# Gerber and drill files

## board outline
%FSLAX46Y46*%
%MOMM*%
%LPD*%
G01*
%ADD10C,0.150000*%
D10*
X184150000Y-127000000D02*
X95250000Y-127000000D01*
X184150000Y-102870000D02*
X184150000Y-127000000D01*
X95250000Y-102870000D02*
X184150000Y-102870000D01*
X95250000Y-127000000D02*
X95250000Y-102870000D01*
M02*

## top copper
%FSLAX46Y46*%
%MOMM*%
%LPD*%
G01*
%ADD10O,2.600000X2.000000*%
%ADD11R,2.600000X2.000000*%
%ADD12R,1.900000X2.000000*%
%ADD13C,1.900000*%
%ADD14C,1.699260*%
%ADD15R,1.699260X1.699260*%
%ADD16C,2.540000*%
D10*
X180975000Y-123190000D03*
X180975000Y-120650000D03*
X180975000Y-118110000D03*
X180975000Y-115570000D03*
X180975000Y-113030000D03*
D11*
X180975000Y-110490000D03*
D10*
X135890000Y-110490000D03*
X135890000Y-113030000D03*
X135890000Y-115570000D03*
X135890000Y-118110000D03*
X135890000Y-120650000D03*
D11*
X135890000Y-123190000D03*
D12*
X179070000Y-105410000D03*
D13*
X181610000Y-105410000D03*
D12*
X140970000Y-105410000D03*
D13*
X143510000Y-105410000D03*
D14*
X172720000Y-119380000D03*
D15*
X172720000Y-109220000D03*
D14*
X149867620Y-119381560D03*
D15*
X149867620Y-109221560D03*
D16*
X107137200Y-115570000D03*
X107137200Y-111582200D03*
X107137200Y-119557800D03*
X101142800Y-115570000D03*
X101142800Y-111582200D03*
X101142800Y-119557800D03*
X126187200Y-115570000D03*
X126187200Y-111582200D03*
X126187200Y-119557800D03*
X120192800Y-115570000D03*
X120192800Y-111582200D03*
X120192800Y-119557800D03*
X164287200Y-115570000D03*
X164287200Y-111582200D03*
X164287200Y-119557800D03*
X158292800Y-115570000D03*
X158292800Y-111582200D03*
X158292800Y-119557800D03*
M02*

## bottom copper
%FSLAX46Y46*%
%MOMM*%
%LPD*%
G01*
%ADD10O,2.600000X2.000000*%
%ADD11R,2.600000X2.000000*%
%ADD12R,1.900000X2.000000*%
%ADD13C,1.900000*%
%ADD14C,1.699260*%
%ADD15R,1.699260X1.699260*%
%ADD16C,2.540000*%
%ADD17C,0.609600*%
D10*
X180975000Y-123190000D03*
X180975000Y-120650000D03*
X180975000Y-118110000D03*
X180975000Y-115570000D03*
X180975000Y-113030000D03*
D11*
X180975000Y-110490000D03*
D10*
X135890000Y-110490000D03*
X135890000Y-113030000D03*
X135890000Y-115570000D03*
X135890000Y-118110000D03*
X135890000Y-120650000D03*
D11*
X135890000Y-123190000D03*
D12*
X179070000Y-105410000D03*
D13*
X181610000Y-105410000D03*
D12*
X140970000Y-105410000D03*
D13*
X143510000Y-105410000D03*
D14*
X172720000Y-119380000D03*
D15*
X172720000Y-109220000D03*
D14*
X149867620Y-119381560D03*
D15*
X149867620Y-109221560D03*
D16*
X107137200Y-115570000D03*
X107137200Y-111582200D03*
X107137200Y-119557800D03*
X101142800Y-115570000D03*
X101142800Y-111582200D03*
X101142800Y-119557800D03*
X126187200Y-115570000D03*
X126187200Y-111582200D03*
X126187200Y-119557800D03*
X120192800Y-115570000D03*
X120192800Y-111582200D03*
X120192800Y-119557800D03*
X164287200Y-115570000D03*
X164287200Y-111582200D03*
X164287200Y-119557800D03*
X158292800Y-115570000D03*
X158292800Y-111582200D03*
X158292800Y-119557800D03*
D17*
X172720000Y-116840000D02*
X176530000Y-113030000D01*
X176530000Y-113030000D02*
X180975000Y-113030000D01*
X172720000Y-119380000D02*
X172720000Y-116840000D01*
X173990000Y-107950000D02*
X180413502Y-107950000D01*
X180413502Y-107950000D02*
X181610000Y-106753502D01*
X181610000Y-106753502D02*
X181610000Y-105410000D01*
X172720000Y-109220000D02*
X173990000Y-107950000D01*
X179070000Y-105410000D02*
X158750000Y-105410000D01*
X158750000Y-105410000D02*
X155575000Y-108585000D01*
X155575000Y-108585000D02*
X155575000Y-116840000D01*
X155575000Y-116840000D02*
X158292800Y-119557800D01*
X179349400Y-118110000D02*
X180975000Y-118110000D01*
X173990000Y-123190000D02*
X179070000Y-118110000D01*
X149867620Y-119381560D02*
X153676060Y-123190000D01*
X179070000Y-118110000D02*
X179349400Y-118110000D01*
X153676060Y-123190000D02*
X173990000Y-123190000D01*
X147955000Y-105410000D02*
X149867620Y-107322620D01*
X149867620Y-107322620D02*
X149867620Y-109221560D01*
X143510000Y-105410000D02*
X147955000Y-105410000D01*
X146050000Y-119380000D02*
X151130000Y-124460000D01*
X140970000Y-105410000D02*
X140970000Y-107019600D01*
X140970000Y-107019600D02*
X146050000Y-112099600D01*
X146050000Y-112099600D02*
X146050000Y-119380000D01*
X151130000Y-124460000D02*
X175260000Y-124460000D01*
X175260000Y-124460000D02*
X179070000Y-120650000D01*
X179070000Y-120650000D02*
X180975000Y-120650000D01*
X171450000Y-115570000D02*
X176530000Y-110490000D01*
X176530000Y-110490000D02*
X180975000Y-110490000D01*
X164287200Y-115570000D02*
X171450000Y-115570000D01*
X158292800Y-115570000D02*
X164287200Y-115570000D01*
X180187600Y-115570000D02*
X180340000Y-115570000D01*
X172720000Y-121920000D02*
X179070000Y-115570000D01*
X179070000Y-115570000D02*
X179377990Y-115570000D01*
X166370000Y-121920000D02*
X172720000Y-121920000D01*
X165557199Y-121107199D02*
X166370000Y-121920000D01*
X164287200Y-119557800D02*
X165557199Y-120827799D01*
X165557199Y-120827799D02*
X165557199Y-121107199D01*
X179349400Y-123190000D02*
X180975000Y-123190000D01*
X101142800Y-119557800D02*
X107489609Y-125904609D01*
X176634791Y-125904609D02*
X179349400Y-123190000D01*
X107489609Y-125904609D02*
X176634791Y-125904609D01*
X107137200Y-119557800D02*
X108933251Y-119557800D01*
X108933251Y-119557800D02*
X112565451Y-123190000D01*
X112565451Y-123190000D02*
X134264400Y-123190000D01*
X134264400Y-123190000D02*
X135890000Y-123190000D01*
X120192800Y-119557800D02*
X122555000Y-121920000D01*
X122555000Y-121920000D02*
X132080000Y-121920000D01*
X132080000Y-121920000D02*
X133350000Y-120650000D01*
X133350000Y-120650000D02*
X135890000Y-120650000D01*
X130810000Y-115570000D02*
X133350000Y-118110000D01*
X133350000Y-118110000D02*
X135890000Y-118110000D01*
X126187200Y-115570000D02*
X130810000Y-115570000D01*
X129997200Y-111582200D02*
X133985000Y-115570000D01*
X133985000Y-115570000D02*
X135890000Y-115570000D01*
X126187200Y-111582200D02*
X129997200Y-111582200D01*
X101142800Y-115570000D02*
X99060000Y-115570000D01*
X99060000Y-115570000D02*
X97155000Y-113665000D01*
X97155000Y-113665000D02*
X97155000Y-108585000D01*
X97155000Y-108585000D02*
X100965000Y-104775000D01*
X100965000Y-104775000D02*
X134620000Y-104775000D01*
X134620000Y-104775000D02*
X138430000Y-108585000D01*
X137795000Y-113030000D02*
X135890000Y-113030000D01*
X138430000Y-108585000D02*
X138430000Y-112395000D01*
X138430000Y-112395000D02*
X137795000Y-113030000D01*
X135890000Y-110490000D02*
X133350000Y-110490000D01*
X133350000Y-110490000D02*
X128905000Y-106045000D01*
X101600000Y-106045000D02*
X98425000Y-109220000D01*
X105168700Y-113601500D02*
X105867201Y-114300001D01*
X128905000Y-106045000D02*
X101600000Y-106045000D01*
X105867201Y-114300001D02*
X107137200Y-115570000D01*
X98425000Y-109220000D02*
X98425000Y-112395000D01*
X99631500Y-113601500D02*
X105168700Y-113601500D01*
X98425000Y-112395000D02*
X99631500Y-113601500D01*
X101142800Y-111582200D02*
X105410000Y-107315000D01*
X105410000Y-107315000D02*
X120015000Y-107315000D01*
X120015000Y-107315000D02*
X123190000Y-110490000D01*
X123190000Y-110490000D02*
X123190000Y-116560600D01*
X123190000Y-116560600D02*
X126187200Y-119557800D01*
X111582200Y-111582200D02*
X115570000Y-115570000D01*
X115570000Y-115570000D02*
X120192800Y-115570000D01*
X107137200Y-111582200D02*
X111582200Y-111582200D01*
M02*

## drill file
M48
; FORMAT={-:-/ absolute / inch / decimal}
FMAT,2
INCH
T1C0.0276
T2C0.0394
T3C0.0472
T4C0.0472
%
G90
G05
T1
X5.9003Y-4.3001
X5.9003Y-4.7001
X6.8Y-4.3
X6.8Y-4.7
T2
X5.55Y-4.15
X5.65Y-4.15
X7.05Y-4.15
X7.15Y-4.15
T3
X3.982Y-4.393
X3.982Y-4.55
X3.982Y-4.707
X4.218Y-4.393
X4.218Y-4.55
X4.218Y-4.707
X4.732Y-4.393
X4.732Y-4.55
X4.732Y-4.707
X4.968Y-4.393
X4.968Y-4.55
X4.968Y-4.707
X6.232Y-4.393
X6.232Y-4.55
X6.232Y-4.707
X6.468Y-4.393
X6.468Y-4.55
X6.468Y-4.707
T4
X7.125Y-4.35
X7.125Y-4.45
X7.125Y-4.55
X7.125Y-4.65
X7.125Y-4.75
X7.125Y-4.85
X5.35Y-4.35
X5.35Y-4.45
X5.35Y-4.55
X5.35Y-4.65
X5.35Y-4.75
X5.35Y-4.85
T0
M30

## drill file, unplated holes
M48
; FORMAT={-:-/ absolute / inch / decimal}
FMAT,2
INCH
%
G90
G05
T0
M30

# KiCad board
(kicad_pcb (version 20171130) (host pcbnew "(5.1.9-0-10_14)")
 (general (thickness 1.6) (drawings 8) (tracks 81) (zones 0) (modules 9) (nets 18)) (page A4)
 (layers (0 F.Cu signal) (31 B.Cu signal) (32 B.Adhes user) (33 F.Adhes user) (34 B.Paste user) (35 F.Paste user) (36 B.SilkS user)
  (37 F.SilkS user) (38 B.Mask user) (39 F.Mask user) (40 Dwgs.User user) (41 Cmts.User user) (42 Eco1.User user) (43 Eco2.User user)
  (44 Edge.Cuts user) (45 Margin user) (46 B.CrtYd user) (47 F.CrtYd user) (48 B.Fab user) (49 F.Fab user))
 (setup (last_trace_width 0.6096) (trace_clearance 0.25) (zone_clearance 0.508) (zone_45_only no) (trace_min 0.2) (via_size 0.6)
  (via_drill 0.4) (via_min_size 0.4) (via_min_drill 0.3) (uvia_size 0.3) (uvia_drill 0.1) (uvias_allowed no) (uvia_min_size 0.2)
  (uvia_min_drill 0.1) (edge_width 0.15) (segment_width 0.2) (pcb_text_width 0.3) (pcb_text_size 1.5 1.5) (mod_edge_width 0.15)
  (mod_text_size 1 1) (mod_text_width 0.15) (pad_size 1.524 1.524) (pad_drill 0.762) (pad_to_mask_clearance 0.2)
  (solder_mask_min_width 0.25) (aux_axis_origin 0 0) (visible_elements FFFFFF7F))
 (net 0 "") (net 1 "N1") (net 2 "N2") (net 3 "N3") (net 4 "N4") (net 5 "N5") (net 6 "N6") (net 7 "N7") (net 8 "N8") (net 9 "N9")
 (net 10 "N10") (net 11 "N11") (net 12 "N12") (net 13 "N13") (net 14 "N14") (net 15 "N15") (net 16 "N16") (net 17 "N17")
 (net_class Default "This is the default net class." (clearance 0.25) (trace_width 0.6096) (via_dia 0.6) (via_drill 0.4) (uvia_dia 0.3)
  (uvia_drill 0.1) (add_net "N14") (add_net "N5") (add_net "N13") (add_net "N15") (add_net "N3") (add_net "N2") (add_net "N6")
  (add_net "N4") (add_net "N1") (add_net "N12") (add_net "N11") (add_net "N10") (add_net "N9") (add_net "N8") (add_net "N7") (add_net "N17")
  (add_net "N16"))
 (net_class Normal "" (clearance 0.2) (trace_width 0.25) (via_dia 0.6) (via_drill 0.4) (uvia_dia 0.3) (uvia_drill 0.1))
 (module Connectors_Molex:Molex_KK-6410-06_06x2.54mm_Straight (layer F.Cu) (at 180.975 110.49 270)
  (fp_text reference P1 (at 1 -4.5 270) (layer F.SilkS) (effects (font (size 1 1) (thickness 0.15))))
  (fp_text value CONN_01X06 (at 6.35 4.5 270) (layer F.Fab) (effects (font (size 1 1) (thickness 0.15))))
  (pad 6 thru_hole oval (at 12.7 0 270) (size 2 2.6) (drill 1.2) (layers *.Cu *.Mask) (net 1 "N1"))
  (pad 5 thru_hole oval (at 10.16 0 270) (size 2 2.6) (drill 1.2) (layers *.Cu *.Mask) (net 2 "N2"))
  (pad 4 thru_hole oval (at 7.62 0 270) (size 2 2.6) (drill 1.2) (layers *.Cu *.Mask) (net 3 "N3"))
  (pad 3 thru_hole oval (at 5.08 0 270) (size 2 2.6) (drill 1.2) (layers *.Cu *.Mask) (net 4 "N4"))
  (pad 2 thru_hole oval (at 2.54 0 270) (size 2 2.6) (drill 1.2) (layers *.Cu *.Mask) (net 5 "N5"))
  (pad 1 thru_hole rect (at 0 0 270) (size 2 2.6) (drill 1.2) (layers *.Cu *.Mask) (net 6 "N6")))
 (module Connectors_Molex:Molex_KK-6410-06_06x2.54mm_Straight (layer F.Cu) (at 135.89 123.19 90)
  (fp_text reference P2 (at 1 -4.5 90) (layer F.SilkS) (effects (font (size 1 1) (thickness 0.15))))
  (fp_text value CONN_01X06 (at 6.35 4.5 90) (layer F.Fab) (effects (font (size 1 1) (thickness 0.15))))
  (pad 6 thru_hole oval (at 12.7 0 90) (size 2 2.6) (drill 1.2) (layers *.Cu *.Mask) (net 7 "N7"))
  (pad 5 thru_hole oval (at 10.16 0 90) (size 2 2.6) (drill 1.2) (layers *.Cu *.Mask) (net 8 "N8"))
  (pad 4 thru_hole oval (at 7.62 0 90) (size 2 2.6) (drill 1.2) (layers *.Cu *.Mask) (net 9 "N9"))
  (pad 3 thru_hole oval (at 5.08 0 90) (size 2 2.6) (drill 1.2) (layers *.Cu *.Mask) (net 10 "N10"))
  (pad 2 thru_hole oval (at 2.54 0 90) (size 2 2.6) (drill 1.2) (layers *.Cu *.Mask) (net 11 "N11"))
  (pad 1 thru_hole rect (at 0 0 90) (size 2 2.6) (drill 1.2) (layers *.Cu *.Mask) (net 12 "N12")))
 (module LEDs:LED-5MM (layer F.Cu) (at 179.07 105.41)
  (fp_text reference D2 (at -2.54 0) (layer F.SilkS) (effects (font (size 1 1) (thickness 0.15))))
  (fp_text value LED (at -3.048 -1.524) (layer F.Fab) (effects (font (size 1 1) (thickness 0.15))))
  (pad 1 thru_hole rect (at 0 0 90) (size 2 1.9) (drill 1.00076) (layers *.Cu *.Mask F.SilkS) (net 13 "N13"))
  (pad 2 thru_hole circle (at 2.54 0) (size 1.9 1.9) (drill 1.00076) (layers *.Cu *.Mask F.SilkS) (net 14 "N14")))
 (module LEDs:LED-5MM (layer F.Cu) (at 140.97 105.41)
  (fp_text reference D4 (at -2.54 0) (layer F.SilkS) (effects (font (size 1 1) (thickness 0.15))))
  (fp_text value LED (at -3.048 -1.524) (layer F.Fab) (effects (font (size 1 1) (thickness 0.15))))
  (pad 1 thru_hole rect (at 0 0 90) (size 2 1.9) (drill 1.00076) (layers *.Cu *.Mask F.SilkS) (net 2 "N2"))
  (pad 2 thru_hole circle (at 2.54 0) (size 1.9 1.9) (drill 1.00076) (layers *.Cu *.Mask F.SilkS) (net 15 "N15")))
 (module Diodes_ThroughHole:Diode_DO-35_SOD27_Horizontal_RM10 (layer F.Cu) (at 172.71746 109.21948 270)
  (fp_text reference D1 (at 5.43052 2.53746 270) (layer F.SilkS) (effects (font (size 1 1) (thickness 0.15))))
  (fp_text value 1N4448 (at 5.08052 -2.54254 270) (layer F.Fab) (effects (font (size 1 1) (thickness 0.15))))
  (pad 2 thru_hole circle (at 10.16052 -0.00254 90) (size 1.69926 1.69926) (drill 0.70104) (layers *.Cu *.Mask F.SilkS) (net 5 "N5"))
  (pad 1 thru_hole rect (at 0.00052 -0.00254 90) (size 1.69926 1.69926) (drill 0.70104) (layers *.Cu *.Mask F.SilkS) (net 14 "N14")))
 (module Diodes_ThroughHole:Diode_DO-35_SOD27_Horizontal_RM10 (layer F.Cu) (at 149.86508 109.22104 270)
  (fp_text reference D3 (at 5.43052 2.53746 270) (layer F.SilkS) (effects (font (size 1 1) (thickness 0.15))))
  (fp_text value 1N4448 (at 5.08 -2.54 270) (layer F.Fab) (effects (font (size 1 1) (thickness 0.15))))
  (pad 2 thru_hole circle (at 10.16052 -0.00254 90) (size 1.69926 1.69926) (drill 0.70104) (layers *.Cu *.Mask F.SilkS) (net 3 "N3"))
  (pad 1 thru_hole rect (at 0.00052 -0.00254 90) (size 1.69926 1.69926) (drill 0.70104) (layers *.Cu *.Mask F.SilkS) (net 15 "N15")))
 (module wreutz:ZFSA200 (layer F.Cu) (at 104.14 115.57 270)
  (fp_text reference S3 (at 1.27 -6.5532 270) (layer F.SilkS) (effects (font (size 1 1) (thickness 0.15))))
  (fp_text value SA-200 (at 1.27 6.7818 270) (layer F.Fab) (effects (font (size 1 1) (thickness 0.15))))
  (pad 10 thru_hole circle (at 0 -2.9972 270) (size 2.54 2.54) (drill 1.19888) (layers *.Cu *.Mask F.SilkS) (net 7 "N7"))
  (pad 11 thru_hole circle (at -3.9878 -2.9972 270) (size 2.54 2.54) (drill 1.19888) (layers *.Cu *.Mask F.SilkS) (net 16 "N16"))
  (pad 12 thru_hole circle (at 3.9878 -2.9972 270) (size 2.54 2.54) (drill 1.19888) (layers *.Cu *.Mask F.SilkS) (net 12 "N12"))
  (pad 20 thru_hole circle (at 0 2.9972 270) (size 2.54 2.54) (drill 1.19888) (layers *.Cu *.Mask F.SilkS) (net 8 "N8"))
  (pad 21 thru_hole circle (at -3.9878 2.9972 270) (size 2.54 2.54) (drill 1.19888) (layers *.Cu *.Mask F.SilkS) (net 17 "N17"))
  (pad 22 thru_hole circle (at 3.9878 2.9972 270) (size 2.54 2.54) (drill 1.19888) (layers *.Cu *.Mask F.SilkS) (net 1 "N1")))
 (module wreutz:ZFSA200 (layer F.Cu) (at 123.19 115.57 270)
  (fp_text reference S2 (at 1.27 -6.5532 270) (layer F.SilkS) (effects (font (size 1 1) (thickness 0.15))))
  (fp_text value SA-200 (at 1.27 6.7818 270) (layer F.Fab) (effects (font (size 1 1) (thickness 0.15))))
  (pad 10 thru_hole circle (at 0 -2.9972 270) (size 2.54 2.54) (drill 1.19888) (layers *.Cu *.Mask F.SilkS) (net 10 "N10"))
  (pad 11 thru_hole circle (at -3.9878 -2.9972 270) (size 2.54 2.54) (drill 1.19888) (layers *.Cu *.Mask F.SilkS) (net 9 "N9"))
  (pad 12 thru_hole circle (at 3.9878 -2.9972 270) (size 2.54 2.54) (drill 1.19888) (layers *.Cu *.Mask F.SilkS) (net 17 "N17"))
  (pad 20 thru_hole circle (at 0 2.9972 270) (size 2.54 2.54) (drill 1.19888) (layers *.Cu *.Mask F.SilkS) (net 16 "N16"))
  (pad 21 thru_hole circle (at -3.9878 2.9972 270) (size 2.54 2.54) (drill 1.19888) (layers *.Cu *.Mask F.SilkS))
  (pad 22 thru_hole circle (at 3.9878 2.9972 270) (size 2.54 2.54) (drill 1.19888) (layers *.Cu *.Mask F.SilkS) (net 11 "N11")))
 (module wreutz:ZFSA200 (layer F.Cu) (at 161.29 115.57 270)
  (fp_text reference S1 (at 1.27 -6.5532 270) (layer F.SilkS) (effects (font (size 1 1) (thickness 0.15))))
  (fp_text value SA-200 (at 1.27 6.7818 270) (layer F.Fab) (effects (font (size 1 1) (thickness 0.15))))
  (pad 10 thru_hole circle (at 0 -2.9972 270) (size 2.54 2.54) (drill 1.19888) (layers *.Cu *.Mask F.SilkS) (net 6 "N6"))
  (pad 11 thru_hole circle (at -3.9878 -2.9972 270) (size 2.54 2.54) (drill 1.19888) (layers *.Cu *.Mask F.SilkS))
  (pad 12 thru_hole circle (at 3.9878 -2.9972 270) (size 2.54 2.54) (drill 1.19888) (layers *.Cu *.Mask F.SilkS) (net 4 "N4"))
  (pad 20 thru_hole circle (at 0 2.9972 270) (size 2.54 2.54) (drill 1.19888) (layers *.Cu *.Mask F.SilkS) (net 6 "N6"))
  (pad 21 thru_hole circle (at -3.9878 2.9972 270) (size 2.54 2.54) (drill 1.19888) (layers *.Cu *.Mask F.SilkS))
  (pad 22 thru_hole circle (at 3.9878 2.9972 270) (size 2.54 2.54) (drill 1.19888) (layers *.Cu *.Mask F.SilkS) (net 13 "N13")))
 (gr_line (start 184.15 127) (end 95.25 127) (layer Edge.Cuts) (width 0.15))
 (gr_line (start 184.15 102.87) (end 184.15 127) (layer Edge.Cuts) (width 0.15))
 (gr_line (start 95.25 102.87) (end 184.15 102.87) (layer Edge.Cuts) (width 0.15))
 (gr_line (start 95.25 127) (end 95.25 102.87) (layer Edge.Cuts) (width 0.15))
 (segment (start 172.72 116.84) (end 176.53 113.03) (width 0.6096) (layer B.Cu) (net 5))
 (segment (start 176.53 113.03) (end 180.975 113.03) (width 0.6096) (layer B.Cu) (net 5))
 (segment (start 172.72 119.38) (end 172.72 116.84) (width 0.6096) (layer B.Cu) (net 5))
 (segment (start 173.99 107.95) (end 180.413502 107.95) (width 0.6096) (layer B.Cu) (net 14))
 (segment (start 180.413502 107.95) (end 181.61 106.753502) (width 0.6096) (layer B.Cu) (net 14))
 (segment (start 181.61 106.753502) (end 181.61 105.41) (width 0.6096) (layer B.Cu) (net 14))
 (segment (start 172.72 109.22) (end 173.99 107.95) (width 0.6096) (layer B.Cu) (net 14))
 (segment (start 179.07 105.41) (end 158.75 105.41) (width 0.6096) (layer B.Cu) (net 13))
 (segment (start 158.75 105.41) (end 155.575 108.585) (width 0.6096) (layer B.Cu) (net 13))
 (segment (start 155.575 108.585) (end 155.575 116.84) (width 0.6096) (layer B.Cu) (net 13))
 (segment (start 155.575 116.84) (end 158.2928 119.5578) (width 0.6096) (layer B.Cu) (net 13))
 (segment (start 179.3494 118.11) (end 180.975 118.11) (width 0.6096) (layer B.Cu) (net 3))
 (segment (start 173.99 123.19) (end 179.07 118.11) (width 0.6096) (layer B.Cu) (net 3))
 (segment (start 149.86762 119.38156) (end 153.67606 123.19) (width 0.6096) (layer B.Cu) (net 3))
 (segment (start 179.07 118.11) (end 179.3494 118.11) (width 0.6096) (layer B.Cu) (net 3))
 (segment (start 153.67606 123.19) (end 173.99 123.19) (width 0.6096) (layer B.Cu) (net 3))
 (segment (start 147.955 105.41) (end 149.86762 107.32262) (width 0.6096) (layer B.Cu) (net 15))
 (segment (start 149.86762 107.32262) (end 149.86762 109.22156) (width 0.6096) (layer B.Cu) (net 15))
 (segment (start 143.51 105.41) (end 147.955 105.41) (width 0.6096) (layer B.Cu) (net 15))
 (segment (start 146.05 119.38) (end 151.13 124.46) (width 0.6096) (layer B.Cu) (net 2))
 (segment (start 140.97 105.41) (end 140.97 107.0196) (width 0.6096) (layer B.Cu) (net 2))
 (segment (start 140.97 107.0196) (end 146.05 112.0996) (width 0.6096) (layer B.Cu) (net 2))
 (segment (start 146.05 112.0996) (end 146.05 119.38) (width 0.6096) (layer B.Cu) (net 2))
 (segment (start 151.13 124.46) (end 175.26 124.46) (width 0.6096) (layer B.Cu) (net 2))
 (segment (start 175.26 124.46) (end 179.07 120.65) (width 0.6096) (layer B.Cu) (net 2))
 (segment (start 179.07 120.65) (end 180.975 120.65) (width 0.6096) (layer B.Cu) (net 2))
 (segment (start 171.45 115.57) (end 176.53 110.49) (width 0.6096) (layer B.Cu) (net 6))
 (segment (start 176.53 110.49) (end 180.975 110.49) (width 0.6096) (layer B.Cu) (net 6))
 (segment (start 164.2872 115.57) (end 171.45 115.57) (width 0.6096) (layer B.Cu) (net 6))
 (segment (start 158.2928 115.57) (end 164.2872 115.57) (width 0.6096) (layer B.Cu) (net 6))
 (segment (start 180.1876 115.57) (end 180.34 115.57) (width 0.6096) (layer B.Cu) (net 4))
 (segment (start 172.72 121.92) (end 179.07 115.57) (width 0.6096) (layer B.Cu) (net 4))
 (segment (start 179.07 115.57) (end 179.37799 115.57) (width 0.6096) (layer B.Cu) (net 4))
 (segment (start 166.37 121.92) (end 172.72 121.92) (width 0.6096) (layer B.Cu) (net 4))
 (segment (start 165.557199 121.107199) (end 166.37 121.92) (width 0.6096) (layer B.Cu) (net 4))
 (segment (start 164.2872 119.5578) (end 165.557199 120.827799) (width 0.6096) (layer B.Cu) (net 4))
 (segment (start 165.557199 120.827799) (end 165.557199 121.107199) (width 0.6096) (layer B.Cu) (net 4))
 (segment (start 179.3494 123.19) (end 180.975 123.19) (width 0.6096) (layer B.Cu) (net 1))
 (segment (start 101.1428 119.5578) (end 107.489609 125.904609) (width 0.6096) (layer B.Cu) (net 1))
 (segment (start 176.634791 125.904609) (end 179.3494 123.19) (width 0.6096) (layer B.Cu) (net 1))
 (segment (start 107.489609 125.904609) (end 176.634791 125.904609) (width 0.6096) (layer B.Cu) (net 1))
 (segment (start 107.1372 119.5578) (end 108.933251 119.5578) (width 0.6096) (layer B.Cu) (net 12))
 (segment (start 108.933251 119.5578) (end 112.565451 123.19) (width 0.6096) (layer B.Cu) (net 12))
 (segment (start 112.565451 123.19) (end 134.2644 123.19) (width 0.6096) (layer B.Cu) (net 12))
 (segment (start 134.2644 123.19) (end 135.89 123.19) (width 0.6096) (layer B.Cu) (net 12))
 (segment (start 120.1928 119.5578) (end 122.555 121.92) (width 0.6096) (layer B.Cu) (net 11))
 (segment (start 122.555 121.92) (end 132.08 121.92) (width 0.6096) (layer B.Cu) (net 11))
 (segment (start 132.08 121.92) (end 133.35 120.65) (width 0.6096) (layer B.Cu) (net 11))
 (segment (start 133.35 120.65) (end 135.89 120.65) (width 0.6096) (layer B.Cu) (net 11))
 (segment (start 130.81 115.57) (end 133.35 118.11) (width 0.6096) (layer B.Cu) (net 10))
 (segment (start 133.35 118.11) (end 135.89 118.11) (width 0.6096) (layer B.Cu) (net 10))
 (segment (start 126.1872 115.57) (end 130.81 115.57) (width 0.6096) (layer B.Cu) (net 10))
 (segment (start 129.9972 111.5822) (end 133.985 115.57) (width 0.6096) (layer B.Cu) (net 9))
 (segment (start 133.985 115.57) (end 135.89 115.57) (width 0.6096) (layer B.Cu) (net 9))
 (segment (start 126.1872 111.5822) (end 129.9972 111.5822) (width 0.6096) (layer B.Cu) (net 9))
 (segment (start 101.1428 115.57) (end 99.06 115.57) (width 0.6096) (layer B.Cu) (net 8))
 (segment (start 99.06 115.57) (end 97.155 113.665) (width 0.6096) (layer B.Cu) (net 8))
 (segment (start 97.155 113.665) (end 97.155 108.585) (width 0.6096) (layer B.Cu) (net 8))
 (segment (start 97.155 108.585) (end 100.965 104.775) (width 0.6096) (layer B.Cu) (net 8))
 (segment (start 100.965 104.775) (end 134.62 104.775) (width 0.6096) (layer B.Cu) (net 8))
 (segment (start 134.62 104.775) (end 138.43 108.585) (width 0.6096) (layer B.Cu) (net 8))
 (segment (start 137.795 113.03) (end 135.89 113.03) (width 0.6096) (layer B.Cu) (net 8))
 (segment (start 138.43 108.585) (end 138.43 112.395) (width 0.6096) (layer B.Cu) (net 8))
 (segment (start 138.43 112.395) (end 137.795 113.03) (width 0.6096) (layer B.Cu) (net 8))
 (segment (start 135.89 110.49) (end 133.35 110.49) (width 0.6096) (layer B.Cu) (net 7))
 (segment (start 133.35 110.49) (end 128.905 106.045) (width 0.6096) (layer B.Cu) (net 7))
 (segment (start 101.6 106.045) (end 98.425 109.22) (width 0.6096) (layer B.Cu) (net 7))
 (segment (start 105.1687 113.6015) (end 105.867201 114.300001) (width 0.6096) (layer B.Cu) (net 7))
 (segment (start 128.905 106.045) (end 101.6 106.045) (width 0.6096) (layer B.Cu) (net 7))
 (segment (start 105.867201 114.300001) (end 107.1372 115.57) (width 0.6096) (layer B.Cu) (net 7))
 (segment (start 98.425 109.22) (end 98.425 112.395) (width 0.6096) (layer B.Cu) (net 7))
 (segment (start 99.6315 113.6015) (end 105.1687 113.6015) (width 0.6096) (layer B.Cu) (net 7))
 (segment (start 98.425 112.395) (end 99.6315 113.6015) (width 0.6096) (layer B.Cu) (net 7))
 (segment (start 101.1428 111.5822) (end 105.41 107.315) (width 0.6096) (layer B.Cu) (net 17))
 (segment (start 105.41 107.315) (end 120.015 107.315) (width 0.6096) (layer B.Cu) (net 17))
 (segment (start 120.015 107.315) (end 123.19 110.49) (width 0.6096) (layer B.Cu) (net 17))
 (segment (start 123.19 110.49) (end 123.19 116.5606) (width 0.6096) (layer B.Cu) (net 17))
 (segment (start 123.19 116.5606) (end 126.1872 119.5578) (width 0.6096) (layer B.Cu) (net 17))
 (segment (start 111.5822 111.5822) (end 115.57 115.57) (width 0.6096) (layer B.Cu) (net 16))
 (segment (start 115.57 115.57) (end 120.1928 115.57) (width 0.6096) (layer B.Cu) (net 16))
 (segment (start 107.1372 111.5822) (end 111.5822 111.5822) (width 0.6096) (layer B.Cu) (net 16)))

